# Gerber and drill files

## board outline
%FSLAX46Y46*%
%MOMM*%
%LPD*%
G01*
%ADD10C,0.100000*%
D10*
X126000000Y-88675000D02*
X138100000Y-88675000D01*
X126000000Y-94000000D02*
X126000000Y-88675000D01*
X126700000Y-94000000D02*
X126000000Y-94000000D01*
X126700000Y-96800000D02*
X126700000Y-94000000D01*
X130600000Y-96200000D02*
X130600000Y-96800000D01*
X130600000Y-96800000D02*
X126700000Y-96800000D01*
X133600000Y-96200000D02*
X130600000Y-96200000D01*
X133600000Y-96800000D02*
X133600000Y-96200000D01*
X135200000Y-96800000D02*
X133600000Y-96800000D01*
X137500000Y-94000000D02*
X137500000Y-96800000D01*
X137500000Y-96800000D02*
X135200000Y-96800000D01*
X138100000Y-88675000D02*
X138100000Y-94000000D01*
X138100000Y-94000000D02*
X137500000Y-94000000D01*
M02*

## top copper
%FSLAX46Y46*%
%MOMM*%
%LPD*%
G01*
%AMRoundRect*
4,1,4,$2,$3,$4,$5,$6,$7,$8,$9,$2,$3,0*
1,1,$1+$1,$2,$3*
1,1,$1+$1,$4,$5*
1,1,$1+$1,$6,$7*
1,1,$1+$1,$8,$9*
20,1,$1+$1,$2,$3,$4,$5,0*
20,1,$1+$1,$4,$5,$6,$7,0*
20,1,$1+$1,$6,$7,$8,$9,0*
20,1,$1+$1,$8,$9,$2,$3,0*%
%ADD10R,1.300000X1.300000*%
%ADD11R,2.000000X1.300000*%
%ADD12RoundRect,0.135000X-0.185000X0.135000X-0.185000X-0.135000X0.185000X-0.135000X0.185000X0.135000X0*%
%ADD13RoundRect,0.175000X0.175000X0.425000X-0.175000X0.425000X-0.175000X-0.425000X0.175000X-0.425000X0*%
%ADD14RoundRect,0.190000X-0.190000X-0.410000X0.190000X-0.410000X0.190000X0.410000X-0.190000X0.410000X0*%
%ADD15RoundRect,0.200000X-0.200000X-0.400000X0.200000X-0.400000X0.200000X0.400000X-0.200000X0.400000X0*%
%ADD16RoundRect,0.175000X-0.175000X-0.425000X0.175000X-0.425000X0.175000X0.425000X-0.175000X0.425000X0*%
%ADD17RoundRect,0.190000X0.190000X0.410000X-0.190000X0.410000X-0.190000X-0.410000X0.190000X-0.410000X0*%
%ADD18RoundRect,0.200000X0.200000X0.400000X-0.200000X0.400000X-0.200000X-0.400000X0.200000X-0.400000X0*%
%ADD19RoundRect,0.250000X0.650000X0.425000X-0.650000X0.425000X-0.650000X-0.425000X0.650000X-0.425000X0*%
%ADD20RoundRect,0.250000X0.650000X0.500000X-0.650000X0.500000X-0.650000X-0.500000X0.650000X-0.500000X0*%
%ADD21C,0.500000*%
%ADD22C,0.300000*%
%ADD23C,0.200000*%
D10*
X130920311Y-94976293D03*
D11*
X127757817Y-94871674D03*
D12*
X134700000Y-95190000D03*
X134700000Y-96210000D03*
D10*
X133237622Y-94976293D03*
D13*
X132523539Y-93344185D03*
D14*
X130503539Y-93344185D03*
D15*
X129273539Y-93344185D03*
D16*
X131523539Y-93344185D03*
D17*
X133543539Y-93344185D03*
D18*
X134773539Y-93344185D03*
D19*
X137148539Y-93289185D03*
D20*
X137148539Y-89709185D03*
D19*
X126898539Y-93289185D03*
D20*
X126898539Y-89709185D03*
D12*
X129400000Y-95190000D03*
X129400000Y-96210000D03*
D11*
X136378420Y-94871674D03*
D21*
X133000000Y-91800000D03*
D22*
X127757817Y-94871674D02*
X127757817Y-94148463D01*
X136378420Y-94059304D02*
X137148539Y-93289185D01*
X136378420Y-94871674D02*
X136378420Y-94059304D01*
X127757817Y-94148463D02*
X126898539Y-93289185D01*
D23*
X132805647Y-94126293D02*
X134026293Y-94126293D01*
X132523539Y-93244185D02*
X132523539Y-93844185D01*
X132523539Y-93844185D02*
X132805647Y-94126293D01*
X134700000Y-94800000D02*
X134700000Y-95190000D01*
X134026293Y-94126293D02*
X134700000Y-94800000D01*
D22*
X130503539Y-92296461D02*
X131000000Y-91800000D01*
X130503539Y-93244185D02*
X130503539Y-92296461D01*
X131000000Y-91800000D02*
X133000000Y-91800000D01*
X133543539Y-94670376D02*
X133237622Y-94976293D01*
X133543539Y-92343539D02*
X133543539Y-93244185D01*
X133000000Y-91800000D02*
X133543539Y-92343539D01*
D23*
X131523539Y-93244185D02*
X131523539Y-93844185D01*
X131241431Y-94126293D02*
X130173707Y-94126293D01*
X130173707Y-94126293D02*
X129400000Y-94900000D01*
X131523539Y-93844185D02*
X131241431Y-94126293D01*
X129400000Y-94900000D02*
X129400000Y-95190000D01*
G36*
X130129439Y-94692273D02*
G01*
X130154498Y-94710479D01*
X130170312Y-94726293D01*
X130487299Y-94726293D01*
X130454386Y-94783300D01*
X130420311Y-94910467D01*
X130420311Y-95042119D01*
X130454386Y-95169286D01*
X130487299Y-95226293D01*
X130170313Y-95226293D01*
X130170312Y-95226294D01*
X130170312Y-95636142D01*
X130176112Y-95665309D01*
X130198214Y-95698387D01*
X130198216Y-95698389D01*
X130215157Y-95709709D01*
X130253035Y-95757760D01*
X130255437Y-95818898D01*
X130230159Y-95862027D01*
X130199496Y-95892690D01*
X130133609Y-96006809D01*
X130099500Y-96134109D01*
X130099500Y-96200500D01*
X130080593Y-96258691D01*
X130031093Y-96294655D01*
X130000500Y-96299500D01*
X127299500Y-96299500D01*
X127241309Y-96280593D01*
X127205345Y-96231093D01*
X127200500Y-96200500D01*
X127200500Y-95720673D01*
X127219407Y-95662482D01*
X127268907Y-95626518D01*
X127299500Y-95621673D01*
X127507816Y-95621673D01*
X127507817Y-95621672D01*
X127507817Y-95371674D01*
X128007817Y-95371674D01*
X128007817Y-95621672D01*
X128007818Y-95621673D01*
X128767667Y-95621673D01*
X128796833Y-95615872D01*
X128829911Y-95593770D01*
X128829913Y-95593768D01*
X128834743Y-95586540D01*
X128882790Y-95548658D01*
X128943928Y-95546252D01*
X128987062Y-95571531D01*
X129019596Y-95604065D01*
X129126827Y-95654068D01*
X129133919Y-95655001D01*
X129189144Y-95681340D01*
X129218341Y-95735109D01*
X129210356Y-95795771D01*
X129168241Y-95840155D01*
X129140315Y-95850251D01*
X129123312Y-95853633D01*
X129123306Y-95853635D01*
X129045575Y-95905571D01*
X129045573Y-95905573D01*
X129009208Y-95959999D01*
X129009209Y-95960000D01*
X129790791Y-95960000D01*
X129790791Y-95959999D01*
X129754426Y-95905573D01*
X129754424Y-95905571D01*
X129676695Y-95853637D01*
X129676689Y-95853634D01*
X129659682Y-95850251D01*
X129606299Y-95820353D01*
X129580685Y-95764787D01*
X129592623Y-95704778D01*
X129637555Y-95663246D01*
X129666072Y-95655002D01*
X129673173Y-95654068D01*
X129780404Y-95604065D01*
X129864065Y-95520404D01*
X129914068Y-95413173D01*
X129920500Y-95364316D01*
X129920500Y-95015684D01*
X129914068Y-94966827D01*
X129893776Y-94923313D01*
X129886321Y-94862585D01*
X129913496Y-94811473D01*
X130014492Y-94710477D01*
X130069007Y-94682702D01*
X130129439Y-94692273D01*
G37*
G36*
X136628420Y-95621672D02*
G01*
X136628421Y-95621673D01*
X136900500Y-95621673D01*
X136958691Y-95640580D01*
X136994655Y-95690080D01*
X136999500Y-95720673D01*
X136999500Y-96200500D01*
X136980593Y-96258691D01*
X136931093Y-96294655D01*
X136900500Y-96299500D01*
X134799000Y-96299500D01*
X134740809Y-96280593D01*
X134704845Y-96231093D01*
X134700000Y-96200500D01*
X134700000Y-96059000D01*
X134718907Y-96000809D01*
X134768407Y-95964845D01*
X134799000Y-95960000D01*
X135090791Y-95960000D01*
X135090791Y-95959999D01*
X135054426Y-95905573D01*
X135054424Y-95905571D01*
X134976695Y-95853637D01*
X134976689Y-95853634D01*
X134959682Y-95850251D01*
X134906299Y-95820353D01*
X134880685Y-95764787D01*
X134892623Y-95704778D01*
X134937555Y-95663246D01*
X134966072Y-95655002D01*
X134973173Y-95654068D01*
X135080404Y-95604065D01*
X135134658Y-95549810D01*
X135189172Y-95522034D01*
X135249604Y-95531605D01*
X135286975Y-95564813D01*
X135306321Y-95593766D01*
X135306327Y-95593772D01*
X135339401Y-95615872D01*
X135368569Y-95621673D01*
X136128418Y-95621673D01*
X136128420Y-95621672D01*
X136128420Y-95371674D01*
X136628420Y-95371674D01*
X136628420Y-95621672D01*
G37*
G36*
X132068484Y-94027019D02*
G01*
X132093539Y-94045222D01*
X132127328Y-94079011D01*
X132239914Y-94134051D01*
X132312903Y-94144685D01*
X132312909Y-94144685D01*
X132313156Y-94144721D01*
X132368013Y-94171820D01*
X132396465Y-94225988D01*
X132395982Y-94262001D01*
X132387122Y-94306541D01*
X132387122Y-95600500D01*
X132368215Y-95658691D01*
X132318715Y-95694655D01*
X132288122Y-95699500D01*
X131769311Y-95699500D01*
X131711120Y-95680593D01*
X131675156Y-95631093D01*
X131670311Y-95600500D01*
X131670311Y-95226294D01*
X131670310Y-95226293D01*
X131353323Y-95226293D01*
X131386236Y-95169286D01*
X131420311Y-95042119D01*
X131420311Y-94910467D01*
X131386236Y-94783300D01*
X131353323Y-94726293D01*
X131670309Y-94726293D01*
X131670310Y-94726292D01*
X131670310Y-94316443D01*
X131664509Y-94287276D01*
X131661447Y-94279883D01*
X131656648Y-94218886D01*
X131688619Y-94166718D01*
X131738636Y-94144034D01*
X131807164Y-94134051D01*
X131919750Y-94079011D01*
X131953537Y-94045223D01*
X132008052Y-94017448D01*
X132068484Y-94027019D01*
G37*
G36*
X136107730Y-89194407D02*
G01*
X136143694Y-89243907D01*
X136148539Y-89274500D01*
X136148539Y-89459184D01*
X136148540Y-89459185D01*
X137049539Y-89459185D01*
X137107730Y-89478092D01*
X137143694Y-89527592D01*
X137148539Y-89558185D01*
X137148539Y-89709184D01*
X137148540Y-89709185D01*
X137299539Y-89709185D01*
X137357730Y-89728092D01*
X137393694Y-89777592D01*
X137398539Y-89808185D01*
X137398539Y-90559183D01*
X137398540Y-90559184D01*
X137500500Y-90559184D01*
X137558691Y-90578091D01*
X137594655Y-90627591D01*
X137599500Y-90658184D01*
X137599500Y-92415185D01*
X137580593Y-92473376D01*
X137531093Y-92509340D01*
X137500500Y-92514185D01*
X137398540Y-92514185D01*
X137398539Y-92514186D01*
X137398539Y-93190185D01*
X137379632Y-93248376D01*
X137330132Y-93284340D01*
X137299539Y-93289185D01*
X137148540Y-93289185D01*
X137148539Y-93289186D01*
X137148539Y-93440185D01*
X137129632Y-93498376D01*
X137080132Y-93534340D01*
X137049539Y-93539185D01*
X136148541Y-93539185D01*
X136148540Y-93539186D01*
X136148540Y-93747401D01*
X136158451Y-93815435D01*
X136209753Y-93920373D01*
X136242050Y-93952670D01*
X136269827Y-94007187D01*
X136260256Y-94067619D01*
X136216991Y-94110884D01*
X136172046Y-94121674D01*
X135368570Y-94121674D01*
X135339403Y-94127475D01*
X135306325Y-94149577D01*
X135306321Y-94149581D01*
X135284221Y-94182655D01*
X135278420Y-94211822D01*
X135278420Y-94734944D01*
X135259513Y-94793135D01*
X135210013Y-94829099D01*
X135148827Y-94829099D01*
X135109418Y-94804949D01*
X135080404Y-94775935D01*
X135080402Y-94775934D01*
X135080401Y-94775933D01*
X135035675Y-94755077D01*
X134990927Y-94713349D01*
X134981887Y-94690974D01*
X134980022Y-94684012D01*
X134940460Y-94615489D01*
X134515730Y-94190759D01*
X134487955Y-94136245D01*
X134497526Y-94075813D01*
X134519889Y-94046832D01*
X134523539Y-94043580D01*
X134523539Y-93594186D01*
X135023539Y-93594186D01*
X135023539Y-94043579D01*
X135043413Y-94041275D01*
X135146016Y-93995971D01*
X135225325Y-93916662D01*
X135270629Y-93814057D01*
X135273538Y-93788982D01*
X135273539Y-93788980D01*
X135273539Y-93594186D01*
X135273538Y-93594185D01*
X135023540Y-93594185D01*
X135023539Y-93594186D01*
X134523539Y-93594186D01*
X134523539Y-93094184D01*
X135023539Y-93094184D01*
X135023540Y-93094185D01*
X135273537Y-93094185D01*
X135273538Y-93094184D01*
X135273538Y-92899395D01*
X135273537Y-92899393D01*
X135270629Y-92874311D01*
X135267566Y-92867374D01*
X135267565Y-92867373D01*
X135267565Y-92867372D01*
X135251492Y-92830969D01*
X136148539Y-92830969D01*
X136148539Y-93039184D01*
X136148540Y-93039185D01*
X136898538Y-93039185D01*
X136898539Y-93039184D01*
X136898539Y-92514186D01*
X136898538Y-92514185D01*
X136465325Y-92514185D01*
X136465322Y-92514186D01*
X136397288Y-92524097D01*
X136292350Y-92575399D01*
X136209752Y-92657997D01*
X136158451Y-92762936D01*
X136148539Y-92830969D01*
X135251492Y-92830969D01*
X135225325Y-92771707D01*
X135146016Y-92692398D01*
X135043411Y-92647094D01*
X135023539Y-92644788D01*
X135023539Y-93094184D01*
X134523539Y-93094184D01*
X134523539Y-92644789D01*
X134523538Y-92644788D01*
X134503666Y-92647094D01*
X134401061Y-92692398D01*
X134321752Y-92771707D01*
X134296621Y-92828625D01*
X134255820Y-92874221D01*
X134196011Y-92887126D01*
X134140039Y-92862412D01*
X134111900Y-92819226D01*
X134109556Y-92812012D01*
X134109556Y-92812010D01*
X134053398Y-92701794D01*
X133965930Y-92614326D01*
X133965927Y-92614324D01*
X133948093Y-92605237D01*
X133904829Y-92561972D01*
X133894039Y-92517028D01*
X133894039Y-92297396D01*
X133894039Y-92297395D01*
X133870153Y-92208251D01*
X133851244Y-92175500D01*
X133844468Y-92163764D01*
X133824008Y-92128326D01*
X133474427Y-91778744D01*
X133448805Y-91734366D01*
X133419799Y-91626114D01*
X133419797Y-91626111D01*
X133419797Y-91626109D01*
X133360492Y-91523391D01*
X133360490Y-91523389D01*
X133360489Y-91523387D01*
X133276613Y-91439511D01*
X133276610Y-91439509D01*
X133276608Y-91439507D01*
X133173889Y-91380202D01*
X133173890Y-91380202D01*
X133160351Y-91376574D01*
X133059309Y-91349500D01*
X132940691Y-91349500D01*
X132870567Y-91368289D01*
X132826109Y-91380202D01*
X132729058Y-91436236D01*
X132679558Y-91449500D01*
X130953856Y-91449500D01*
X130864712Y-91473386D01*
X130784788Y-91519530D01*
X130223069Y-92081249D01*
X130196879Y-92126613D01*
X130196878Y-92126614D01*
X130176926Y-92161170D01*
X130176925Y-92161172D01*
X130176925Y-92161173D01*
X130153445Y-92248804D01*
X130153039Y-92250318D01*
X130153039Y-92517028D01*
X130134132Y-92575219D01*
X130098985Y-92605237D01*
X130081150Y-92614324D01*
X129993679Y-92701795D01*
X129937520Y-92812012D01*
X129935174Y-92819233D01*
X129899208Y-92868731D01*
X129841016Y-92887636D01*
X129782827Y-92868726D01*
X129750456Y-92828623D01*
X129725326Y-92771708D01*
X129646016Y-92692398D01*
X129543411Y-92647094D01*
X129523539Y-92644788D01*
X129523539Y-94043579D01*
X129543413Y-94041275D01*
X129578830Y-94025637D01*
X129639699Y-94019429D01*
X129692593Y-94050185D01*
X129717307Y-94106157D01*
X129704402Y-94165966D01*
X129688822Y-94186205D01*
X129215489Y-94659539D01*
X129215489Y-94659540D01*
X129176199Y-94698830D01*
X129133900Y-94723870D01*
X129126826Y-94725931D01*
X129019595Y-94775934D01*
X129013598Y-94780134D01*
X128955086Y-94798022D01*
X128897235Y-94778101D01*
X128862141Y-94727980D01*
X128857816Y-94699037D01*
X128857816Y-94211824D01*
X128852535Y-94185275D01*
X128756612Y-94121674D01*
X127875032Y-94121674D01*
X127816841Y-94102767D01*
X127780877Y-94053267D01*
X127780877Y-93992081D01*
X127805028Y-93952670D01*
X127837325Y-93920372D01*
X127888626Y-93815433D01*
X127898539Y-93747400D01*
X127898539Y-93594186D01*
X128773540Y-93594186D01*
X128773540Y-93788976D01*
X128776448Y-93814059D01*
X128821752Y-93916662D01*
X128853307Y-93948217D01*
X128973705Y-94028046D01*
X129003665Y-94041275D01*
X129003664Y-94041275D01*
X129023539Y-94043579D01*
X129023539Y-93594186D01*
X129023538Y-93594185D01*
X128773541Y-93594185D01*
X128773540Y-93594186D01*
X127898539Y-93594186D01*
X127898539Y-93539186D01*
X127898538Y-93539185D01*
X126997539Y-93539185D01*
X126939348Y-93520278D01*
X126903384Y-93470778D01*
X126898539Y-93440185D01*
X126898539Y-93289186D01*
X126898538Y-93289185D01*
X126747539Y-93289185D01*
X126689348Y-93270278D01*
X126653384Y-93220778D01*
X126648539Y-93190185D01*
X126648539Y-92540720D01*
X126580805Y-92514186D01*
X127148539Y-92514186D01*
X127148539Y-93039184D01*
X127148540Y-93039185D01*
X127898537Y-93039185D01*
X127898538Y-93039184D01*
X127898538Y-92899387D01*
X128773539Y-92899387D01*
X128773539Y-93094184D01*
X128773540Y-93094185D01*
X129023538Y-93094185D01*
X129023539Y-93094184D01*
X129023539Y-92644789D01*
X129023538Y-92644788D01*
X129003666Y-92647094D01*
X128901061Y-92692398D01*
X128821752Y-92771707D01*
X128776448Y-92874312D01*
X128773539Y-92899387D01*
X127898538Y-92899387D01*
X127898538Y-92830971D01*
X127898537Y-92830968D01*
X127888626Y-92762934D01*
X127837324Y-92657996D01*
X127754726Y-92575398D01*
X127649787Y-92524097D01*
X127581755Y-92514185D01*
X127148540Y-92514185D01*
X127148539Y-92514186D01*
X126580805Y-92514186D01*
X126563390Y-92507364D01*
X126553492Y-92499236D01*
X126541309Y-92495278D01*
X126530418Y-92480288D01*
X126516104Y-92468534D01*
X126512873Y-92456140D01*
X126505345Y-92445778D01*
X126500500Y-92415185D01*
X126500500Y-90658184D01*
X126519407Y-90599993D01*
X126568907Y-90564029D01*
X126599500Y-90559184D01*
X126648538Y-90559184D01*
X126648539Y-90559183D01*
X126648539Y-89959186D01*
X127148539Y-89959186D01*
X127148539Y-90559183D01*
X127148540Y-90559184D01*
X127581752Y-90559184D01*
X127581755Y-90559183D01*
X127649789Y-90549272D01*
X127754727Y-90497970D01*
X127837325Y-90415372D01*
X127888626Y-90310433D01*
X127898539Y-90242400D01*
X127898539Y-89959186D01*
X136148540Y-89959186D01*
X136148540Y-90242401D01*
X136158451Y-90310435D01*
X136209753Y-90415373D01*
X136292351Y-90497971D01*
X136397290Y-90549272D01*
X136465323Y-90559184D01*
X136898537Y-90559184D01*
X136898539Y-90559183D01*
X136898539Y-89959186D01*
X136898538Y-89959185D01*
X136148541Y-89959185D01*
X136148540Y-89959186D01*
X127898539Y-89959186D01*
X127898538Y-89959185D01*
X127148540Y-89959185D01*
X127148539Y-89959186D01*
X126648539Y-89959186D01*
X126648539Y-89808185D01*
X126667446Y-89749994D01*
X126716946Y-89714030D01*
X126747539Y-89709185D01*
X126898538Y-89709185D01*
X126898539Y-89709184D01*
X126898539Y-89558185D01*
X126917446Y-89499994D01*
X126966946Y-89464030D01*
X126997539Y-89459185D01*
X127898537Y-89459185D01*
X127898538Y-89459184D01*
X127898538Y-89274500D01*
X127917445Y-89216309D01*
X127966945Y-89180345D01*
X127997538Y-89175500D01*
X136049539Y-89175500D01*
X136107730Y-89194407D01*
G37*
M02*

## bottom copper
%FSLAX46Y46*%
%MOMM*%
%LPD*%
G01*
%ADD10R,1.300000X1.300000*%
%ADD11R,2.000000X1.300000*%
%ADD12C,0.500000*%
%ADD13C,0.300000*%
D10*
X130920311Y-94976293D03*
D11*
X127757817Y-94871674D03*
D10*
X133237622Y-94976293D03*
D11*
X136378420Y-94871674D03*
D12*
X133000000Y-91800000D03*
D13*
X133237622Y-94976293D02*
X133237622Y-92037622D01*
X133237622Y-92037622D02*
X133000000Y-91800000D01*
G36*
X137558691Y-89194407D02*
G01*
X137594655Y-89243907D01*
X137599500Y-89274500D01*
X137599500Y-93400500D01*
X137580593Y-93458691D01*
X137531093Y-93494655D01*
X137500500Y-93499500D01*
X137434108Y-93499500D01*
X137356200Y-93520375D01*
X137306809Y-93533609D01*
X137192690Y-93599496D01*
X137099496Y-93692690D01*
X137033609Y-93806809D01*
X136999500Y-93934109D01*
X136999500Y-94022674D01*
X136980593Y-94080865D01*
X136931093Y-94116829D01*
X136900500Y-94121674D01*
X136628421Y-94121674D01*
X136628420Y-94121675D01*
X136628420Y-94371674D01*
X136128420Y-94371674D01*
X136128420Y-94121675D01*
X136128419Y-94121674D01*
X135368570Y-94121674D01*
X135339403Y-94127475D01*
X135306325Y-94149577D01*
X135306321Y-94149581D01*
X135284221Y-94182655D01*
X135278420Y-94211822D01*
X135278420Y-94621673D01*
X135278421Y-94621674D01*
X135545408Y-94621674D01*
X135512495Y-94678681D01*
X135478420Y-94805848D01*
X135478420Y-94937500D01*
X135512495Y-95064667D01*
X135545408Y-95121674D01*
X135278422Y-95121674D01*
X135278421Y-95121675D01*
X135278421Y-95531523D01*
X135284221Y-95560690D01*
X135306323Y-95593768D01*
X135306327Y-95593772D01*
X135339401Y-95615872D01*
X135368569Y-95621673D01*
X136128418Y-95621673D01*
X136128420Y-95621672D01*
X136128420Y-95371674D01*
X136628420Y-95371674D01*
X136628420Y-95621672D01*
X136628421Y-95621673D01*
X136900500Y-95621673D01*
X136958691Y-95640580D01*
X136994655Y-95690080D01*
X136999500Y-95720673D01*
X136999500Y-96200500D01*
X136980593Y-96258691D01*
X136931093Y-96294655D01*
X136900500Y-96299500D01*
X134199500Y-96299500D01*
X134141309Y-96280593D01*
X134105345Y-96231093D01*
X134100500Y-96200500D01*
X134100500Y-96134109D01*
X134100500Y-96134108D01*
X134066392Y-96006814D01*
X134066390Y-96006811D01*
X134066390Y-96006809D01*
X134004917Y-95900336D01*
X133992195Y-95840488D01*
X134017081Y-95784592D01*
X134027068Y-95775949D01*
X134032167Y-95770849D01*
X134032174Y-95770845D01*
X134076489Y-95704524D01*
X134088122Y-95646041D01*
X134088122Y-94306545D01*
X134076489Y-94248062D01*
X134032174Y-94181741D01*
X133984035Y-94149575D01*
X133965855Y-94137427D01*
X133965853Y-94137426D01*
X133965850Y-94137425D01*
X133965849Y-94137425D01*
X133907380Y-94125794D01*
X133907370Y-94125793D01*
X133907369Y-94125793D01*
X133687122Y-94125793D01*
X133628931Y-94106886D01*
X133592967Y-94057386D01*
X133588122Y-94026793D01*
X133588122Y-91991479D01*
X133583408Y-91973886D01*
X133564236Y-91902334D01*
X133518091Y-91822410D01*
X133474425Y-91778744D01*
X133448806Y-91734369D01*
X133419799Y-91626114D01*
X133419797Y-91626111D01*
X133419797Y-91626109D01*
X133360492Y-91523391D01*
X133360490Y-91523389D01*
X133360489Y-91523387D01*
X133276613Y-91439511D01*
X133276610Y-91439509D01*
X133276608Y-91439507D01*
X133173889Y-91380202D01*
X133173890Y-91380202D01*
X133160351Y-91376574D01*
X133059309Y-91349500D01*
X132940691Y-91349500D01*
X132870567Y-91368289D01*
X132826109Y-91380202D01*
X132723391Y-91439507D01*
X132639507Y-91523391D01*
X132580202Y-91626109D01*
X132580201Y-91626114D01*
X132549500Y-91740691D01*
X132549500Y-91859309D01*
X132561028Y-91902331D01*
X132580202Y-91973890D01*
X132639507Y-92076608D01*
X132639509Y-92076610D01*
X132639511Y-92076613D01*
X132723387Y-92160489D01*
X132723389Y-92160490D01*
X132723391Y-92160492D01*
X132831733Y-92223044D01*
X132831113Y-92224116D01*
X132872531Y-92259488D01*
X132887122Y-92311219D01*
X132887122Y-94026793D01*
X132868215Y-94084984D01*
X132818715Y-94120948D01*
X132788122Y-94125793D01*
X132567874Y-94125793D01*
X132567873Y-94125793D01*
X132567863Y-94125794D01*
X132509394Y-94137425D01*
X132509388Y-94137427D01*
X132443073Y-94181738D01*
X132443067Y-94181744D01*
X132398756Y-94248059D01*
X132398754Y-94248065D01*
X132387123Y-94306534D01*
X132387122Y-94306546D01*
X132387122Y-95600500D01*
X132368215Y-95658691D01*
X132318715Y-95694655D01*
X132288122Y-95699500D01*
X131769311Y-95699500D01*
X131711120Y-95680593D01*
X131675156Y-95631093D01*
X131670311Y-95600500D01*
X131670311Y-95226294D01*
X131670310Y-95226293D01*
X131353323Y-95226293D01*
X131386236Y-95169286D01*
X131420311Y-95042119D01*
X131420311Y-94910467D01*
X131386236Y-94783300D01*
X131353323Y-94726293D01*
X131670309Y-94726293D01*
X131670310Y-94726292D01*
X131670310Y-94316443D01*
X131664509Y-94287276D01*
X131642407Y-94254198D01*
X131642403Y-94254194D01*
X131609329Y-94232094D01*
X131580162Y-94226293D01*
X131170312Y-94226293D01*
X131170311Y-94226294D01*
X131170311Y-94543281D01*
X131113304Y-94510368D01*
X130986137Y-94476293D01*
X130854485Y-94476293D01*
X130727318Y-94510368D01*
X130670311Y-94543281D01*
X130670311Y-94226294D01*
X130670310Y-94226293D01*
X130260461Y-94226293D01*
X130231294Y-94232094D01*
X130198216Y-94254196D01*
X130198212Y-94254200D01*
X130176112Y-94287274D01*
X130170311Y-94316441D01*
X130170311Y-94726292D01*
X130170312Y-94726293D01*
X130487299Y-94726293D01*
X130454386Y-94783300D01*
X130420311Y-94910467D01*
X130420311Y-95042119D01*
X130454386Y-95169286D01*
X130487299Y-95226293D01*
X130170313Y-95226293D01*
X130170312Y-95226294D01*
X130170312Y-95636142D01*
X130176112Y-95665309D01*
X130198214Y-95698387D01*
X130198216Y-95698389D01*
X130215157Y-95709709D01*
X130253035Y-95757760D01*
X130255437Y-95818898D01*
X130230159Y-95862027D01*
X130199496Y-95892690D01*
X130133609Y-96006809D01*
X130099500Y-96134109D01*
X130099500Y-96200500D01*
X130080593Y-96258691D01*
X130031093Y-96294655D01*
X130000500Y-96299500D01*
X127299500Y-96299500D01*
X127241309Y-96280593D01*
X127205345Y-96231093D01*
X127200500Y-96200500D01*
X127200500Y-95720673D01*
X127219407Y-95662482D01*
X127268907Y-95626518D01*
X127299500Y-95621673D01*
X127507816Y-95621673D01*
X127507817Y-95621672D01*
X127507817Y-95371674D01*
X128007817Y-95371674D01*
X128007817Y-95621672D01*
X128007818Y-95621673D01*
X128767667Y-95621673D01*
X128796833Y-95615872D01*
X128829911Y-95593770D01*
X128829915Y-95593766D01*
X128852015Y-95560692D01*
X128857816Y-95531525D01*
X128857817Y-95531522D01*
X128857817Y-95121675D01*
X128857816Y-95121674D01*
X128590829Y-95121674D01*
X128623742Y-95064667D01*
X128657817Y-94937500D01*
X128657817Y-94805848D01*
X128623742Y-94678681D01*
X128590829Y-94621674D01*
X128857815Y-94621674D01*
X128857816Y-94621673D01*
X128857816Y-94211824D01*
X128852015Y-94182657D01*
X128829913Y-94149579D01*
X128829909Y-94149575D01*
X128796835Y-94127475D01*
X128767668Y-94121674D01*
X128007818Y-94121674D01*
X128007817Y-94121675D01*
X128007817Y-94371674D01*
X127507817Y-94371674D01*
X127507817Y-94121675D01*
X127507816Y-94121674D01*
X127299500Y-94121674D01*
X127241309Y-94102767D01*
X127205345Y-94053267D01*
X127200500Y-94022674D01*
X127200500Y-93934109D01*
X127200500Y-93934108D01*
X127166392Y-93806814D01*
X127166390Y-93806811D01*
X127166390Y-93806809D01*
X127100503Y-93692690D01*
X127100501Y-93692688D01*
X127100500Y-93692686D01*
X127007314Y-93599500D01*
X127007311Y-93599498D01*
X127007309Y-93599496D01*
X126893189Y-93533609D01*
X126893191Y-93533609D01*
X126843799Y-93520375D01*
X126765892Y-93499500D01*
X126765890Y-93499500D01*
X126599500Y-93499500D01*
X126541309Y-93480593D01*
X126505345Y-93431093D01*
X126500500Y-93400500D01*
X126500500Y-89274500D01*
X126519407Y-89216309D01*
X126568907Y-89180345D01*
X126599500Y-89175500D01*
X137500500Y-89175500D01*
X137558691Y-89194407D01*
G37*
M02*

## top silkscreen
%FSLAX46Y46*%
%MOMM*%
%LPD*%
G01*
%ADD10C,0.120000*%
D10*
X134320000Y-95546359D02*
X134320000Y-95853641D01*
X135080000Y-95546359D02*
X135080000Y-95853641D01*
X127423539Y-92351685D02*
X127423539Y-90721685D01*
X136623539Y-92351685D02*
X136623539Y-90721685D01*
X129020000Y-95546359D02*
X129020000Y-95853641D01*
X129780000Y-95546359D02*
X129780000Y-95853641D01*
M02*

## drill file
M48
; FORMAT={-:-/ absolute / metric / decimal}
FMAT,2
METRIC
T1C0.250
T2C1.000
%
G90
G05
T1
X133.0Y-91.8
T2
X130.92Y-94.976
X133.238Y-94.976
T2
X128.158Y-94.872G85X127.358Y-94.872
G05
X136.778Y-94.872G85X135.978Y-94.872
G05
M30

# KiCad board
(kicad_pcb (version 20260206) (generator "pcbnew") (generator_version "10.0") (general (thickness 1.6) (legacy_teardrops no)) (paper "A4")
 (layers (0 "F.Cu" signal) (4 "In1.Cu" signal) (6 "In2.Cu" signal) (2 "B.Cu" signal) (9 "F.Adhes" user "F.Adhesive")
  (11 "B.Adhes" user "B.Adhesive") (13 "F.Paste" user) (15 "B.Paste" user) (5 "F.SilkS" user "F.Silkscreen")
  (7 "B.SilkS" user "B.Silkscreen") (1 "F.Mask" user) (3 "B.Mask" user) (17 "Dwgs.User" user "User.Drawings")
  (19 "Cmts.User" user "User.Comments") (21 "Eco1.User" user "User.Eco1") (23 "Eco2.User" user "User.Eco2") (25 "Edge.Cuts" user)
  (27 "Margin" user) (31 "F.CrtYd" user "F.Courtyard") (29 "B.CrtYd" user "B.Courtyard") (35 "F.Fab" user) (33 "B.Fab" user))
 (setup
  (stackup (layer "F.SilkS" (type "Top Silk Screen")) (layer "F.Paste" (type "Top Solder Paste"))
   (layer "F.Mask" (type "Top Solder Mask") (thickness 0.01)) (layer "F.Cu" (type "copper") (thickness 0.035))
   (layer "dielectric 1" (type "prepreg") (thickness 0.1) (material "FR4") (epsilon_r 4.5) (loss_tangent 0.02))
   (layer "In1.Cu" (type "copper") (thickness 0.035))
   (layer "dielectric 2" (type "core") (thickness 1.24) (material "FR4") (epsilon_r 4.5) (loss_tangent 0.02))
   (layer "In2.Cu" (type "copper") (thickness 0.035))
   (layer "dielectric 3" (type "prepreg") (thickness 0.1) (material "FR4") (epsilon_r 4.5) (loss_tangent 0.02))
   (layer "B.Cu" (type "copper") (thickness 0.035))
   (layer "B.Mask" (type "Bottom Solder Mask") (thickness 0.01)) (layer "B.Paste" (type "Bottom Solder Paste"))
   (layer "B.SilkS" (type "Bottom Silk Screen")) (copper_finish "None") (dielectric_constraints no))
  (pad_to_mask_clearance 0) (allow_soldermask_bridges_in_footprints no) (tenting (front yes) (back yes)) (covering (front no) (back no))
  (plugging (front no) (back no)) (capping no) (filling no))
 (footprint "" (layer "F.Cu") (at 130.920311 94.976293)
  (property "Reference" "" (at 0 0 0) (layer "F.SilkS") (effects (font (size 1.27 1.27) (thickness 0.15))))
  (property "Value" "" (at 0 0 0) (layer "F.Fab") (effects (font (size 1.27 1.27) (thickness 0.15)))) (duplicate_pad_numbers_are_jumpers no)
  (pad "" thru_hole rect (at 0 0 180) (size 1.3 1.3) (drill 1) (layers "*.Cu" "*.Mask") (remove_unused_layers no) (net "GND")))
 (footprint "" (layer "F.Cu") (at 127.757817 94.871674)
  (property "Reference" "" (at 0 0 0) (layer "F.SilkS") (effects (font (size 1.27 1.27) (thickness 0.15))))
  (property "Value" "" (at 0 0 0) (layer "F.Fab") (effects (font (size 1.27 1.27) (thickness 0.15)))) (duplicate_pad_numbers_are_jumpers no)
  (pad "" thru_hole rect (at 0 0 180) (size 2 1.3) (drill oval 1.8 1) (layers "*.Cu" "*.Mask") (remove_unused_layers no) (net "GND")))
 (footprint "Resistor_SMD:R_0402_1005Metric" (layer "F.Cu") (at 134.7 95.7 -90)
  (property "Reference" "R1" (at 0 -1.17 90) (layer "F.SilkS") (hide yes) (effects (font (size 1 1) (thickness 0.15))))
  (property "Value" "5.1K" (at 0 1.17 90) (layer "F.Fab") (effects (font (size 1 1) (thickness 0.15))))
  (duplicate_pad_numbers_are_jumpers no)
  (fp_line (start -0.153641 0.38) (end 0.153641 0.38) (stroke (width 0.12) (type solid)) (layer "F.SilkS"))
  (fp_line (start -0.153641 -0.38) (end 0.153641 -0.38) (stroke (width 0.12) (type solid)) (layer "F.SilkS"))
  (pad "1" smd roundrect (at -0.51 0 270) (size 0.54 0.64) (layers "F.Cu" "F.Mask" "F.Paste") (roundrect_rratio 0.25) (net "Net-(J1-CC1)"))
  (pad "2" smd roundrect (at 0.51 0 270) (size 0.54 0.64) (layers "F.Cu" "F.Mask" "F.Paste") (roundrect_rratio 0.25) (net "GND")))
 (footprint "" (layer "F.Cu") (at 133.237622 94.976293)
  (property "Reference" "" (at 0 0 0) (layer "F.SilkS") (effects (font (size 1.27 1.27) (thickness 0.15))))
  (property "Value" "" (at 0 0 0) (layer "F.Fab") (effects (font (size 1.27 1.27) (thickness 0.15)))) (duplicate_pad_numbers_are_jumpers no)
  (pad "" thru_hole rect (at 0 0 180) (size 1.3 1.3) (drill 1) (layers "*.Cu" "*.Mask") (remove_unused_layers no) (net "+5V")))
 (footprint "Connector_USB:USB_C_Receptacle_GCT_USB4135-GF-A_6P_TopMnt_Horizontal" (layer "F.Cu") (at 132.023539 90.311685 180)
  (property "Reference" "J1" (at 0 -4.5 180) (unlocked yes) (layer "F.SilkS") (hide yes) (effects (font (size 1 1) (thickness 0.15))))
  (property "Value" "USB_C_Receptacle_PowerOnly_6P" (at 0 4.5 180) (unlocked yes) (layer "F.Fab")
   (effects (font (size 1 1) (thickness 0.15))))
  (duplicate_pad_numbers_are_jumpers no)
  (fp_line (start 4.6 -2.04) (end 4.6 -0.41) (stroke (width 0.12) (type solid)) (layer "F.SilkS"))
  (fp_line (start -4.6 -2.04) (end -4.6 -0.41) (stroke (width 0.12) (type solid)) (layer "F.SilkS"))
  (pad "A5" smd roundrect (at -0.5 -3.0325 180) (size 0.7 1.2) (layers "F.Cu" "F.Mask" "F.Paste") (roundrect_rratio 0.25)
   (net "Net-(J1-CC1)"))
  (pad "A9" smd roundrect (at 1.52 -3.0325) (size 0.76 1.2) (layers "F.Cu" "F.Mask" "F.Paste") (roundrect_rratio 0.25) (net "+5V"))
  (pad "A12" smd roundrect (at 2.75 -3.0325) (size 0.8 1.2) (layers "F.Cu" "F.Mask" "F.Paste") (roundrect_rratio 0.25) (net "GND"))
  (pad "B5" smd roundrect (at 0.5 -3.0325) (size 0.7 1.2) (layers "F.Cu" "F.Mask" "F.Paste") (roundrect_rratio 0.25) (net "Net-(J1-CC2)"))
  (pad "B9" smd roundrect (at -1.52 -3.0325 180) (size 0.76 1.2) (layers "F.Cu" "F.Mask" "F.Paste") (roundrect_rratio 0.25) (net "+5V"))
  (pad "B12" smd roundrect (at -2.75 -3.0325 180) (size 0.8 1.2) (layers "F.Cu" "F.Mask" "F.Paste") (roundrect_rratio 0.25) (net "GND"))
  (pad "S1" smd roundrect (at -5.125 -2.9775 180) (size 1.8 1.35) (layers "F.Cu" "F.Mask" "F.Paste") (roundrect_rratio 0.1851851852)
   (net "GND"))
  (pad "S1" smd roundrect (at -5.125 0.6025 180) (size 1.8 1.5) (layers "F.Cu" "F.Mask" "F.Paste") (roundrect_rratio 0.1666666667)
   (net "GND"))
  (pad "S1" smd roundrect (at 5.125 -2.9775 180) (size 1.8 1.35) (layers "F.Cu" "F.Mask" "F.Paste") (roundrect_rratio 0.1851851852)
   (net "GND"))
  (pad "S1" smd roundrect (at 5.125 0.6025 180) (size 1.8 1.5) (layers "F.Cu" "F.Mask" "F.Paste") (roundrect_rratio 0.1666666667)
   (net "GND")))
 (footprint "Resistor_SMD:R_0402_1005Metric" (layer "F.Cu") (at 129.4 95.7 -90)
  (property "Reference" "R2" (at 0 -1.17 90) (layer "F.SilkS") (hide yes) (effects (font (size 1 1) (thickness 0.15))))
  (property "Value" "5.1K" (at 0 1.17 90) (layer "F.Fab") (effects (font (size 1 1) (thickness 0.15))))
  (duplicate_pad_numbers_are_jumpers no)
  (fp_line (start -0.153641 0.38) (end 0.153641 0.38) (stroke (width 0.12) (type solid)) (layer "F.SilkS"))
  (fp_line (start -0.153641 -0.38) (end 0.153641 -0.38) (stroke (width 0.12) (type solid)) (layer "F.SilkS"))
  (pad "1" smd roundrect (at -0.51 0 270) (size 0.54 0.64) (layers "F.Cu" "F.Mask" "F.Paste") (roundrect_rratio 0.25) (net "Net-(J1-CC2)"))
  (pad "2" smd roundrect (at 0.51 0 270) (size 0.54 0.64) (layers "F.Cu" "F.Mask" "F.Paste") (roundrect_rratio 0.25) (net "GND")))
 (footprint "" (layer "F.Cu") (at 136.37842 94.871674)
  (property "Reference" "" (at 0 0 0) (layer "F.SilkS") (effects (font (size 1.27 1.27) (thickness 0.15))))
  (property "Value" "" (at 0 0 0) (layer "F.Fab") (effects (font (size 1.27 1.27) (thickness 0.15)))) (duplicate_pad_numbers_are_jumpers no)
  (pad "" thru_hole rect (at 0 0 180) (size 2 1.3) (drill oval 1.8 1) (layers "*.Cu" "*.Mask") (remove_unused_layers no) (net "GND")))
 (gr_line (start 126 88.675) (end 138.1 88.675) (stroke (width 0.1) (type default)) (layer "Edge.Cuts"))
 (gr_line (start 126 94) (end 126 88.675) (stroke (width 0.1) (type default)) (layer "Edge.Cuts"))
 (gr_line (start 126.7 94) (end 126 94) (stroke (width 0.1) (type default)) (layer "Edge.Cuts"))
 (gr_line (start 126.7 96.8) (end 126.7 94) (stroke (width 0.1) (type default)) (layer "Edge.Cuts"))
 (gr_line (start 130.6 96.2) (end 130.6 96.8) (stroke (width 0.1) (type default)) (layer "Edge.Cuts"))
 (gr_line (start 130.6 96.8) (end 126.7 96.8) (stroke (width 0.1) (type default)) (layer "Edge.Cuts"))
 (gr_line (start 133.6 96.2) (end 130.6 96.2) (stroke (width 0.1) (type default)) (layer "Edge.Cuts"))
 (gr_line (start 133.6 96.8) (end 133.6 96.2) (stroke (width 0.1) (type default)) (layer "Edge.Cuts"))
 (gr_line (start 135.2 96.8) (end 133.6 96.8) (stroke (width 0.1) (type default)) (layer "Edge.Cuts"))
 (gr_line (start 137.5 94) (end 137.5 96.8) (stroke (width 0.1) (type default)) (layer "Edge.Cuts"))
 (gr_line (start 137.5 96.8) (end 135.2 96.8) (stroke (width 0.1) (type default)) (layer "Edge.Cuts"))
 (gr_line (start 138.1 88.675) (end 138.1 94) (stroke (width 0.1) (type default)) (layer "Edge.Cuts"))
 (gr_line (start 138.1 94) (end 137.5 94) (stroke (width 0.1) (type default)) (layer "Edge.Cuts"))
 (segment (start 127.757817 94.871674) (end 127.757817 94.148463) (width 0.3) (layer "F.Cu") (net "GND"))
 (segment (start 136.37842 94.059304) (end 137.148539 93.289185) (width 0.3) (layer "F.Cu") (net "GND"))
 (segment (start 136.37842 94.871674) (end 136.37842 94.059304) (width 0.3) (layer "F.Cu") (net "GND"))
 (segment (start 127.757817 94.148463) (end 126.898539 93.289185) (width 0.3) (layer "F.Cu") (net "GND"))
 (segment (start 132.805647 94.126293) (end 134.026293 94.126293) (width 0.2) (layer "F.Cu") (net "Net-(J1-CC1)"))
 (segment (start 132.523539 93.244185) (end 132.523539 93.844185) (width 0.2) (layer "F.Cu") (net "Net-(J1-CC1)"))
 (segment (start 132.523539 93.844185) (end 132.805647 94.126293) (width 0.2) (layer "F.Cu") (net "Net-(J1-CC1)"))
 (segment (start 134.7 94.8) (end 134.7 95.19) (width 0.2) (layer "F.Cu") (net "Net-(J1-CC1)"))
 (segment (start 134.026293 94.126293) (end 134.7 94.8) (width 0.2) (layer "F.Cu") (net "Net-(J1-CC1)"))
 (segment (start 130.503539 92.296461) (end 131 91.8) (width 0.3) (layer "F.Cu") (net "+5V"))
 (segment (start 130.503539 93.244185) (end 130.503539 92.296461) (width 0.3) (layer "F.Cu") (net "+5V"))
 (segment (start 131 91.8) (end 133 91.8) (width 0.3) (layer "F.Cu") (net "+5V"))
 (segment (start 133.543539 94.670376) (end 133.237622 94.976293) (width 0.3) (layer "F.Cu") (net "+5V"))
 (segment (start 133.543539 92.343539) (end 133.543539 93.244185) (width 0.3) (layer "F.Cu") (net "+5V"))
 (segment (start 133 91.8) (end 133.543539 92.343539) (width 0.3) (layer "F.Cu") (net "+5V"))
 (via (at 133 91.8) (size 0.5) (drill 0.25) (layers "F.Cu" "B.Cu") (capping no) (covering (front no) (back no))
  (plugging (front no) (back no)) (filling no) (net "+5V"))
 (segment (start 133.237622 94.976293) (end 133.237622 92.037622) (width 0.3) (layer "B.Cu") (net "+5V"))
 (segment (start 133.237622 92.037622) (end 133 91.8) (width 0.3) (layer "B.Cu") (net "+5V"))
 (segment (start 131.523539 93.244185) (end 131.523539 93.844185) (width 0.2) (layer "F.Cu") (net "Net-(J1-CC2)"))
 (segment (start 131.241431 94.126293) (end 130.173707 94.126293) (width 0.2) (layer "F.Cu") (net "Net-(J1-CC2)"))
 (segment (start 130.173707 94.126293) (end 129.4 94.9) (width 0.2) (layer "F.Cu") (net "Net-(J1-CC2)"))
 (segment (start 131.523539 93.844185) (end 131.241431 94.126293) (width 0.2) (layer "F.Cu") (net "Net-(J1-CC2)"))
 (segment (start 129.4 94.9) (end 129.4 95.19) (width 0.2) (layer "F.Cu") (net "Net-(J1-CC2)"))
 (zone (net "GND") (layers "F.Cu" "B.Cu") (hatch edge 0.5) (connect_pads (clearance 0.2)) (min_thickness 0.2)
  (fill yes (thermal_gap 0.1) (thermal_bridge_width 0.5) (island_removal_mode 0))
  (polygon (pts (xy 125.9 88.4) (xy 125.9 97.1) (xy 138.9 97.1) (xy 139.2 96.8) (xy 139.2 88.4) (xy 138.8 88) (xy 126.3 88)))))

